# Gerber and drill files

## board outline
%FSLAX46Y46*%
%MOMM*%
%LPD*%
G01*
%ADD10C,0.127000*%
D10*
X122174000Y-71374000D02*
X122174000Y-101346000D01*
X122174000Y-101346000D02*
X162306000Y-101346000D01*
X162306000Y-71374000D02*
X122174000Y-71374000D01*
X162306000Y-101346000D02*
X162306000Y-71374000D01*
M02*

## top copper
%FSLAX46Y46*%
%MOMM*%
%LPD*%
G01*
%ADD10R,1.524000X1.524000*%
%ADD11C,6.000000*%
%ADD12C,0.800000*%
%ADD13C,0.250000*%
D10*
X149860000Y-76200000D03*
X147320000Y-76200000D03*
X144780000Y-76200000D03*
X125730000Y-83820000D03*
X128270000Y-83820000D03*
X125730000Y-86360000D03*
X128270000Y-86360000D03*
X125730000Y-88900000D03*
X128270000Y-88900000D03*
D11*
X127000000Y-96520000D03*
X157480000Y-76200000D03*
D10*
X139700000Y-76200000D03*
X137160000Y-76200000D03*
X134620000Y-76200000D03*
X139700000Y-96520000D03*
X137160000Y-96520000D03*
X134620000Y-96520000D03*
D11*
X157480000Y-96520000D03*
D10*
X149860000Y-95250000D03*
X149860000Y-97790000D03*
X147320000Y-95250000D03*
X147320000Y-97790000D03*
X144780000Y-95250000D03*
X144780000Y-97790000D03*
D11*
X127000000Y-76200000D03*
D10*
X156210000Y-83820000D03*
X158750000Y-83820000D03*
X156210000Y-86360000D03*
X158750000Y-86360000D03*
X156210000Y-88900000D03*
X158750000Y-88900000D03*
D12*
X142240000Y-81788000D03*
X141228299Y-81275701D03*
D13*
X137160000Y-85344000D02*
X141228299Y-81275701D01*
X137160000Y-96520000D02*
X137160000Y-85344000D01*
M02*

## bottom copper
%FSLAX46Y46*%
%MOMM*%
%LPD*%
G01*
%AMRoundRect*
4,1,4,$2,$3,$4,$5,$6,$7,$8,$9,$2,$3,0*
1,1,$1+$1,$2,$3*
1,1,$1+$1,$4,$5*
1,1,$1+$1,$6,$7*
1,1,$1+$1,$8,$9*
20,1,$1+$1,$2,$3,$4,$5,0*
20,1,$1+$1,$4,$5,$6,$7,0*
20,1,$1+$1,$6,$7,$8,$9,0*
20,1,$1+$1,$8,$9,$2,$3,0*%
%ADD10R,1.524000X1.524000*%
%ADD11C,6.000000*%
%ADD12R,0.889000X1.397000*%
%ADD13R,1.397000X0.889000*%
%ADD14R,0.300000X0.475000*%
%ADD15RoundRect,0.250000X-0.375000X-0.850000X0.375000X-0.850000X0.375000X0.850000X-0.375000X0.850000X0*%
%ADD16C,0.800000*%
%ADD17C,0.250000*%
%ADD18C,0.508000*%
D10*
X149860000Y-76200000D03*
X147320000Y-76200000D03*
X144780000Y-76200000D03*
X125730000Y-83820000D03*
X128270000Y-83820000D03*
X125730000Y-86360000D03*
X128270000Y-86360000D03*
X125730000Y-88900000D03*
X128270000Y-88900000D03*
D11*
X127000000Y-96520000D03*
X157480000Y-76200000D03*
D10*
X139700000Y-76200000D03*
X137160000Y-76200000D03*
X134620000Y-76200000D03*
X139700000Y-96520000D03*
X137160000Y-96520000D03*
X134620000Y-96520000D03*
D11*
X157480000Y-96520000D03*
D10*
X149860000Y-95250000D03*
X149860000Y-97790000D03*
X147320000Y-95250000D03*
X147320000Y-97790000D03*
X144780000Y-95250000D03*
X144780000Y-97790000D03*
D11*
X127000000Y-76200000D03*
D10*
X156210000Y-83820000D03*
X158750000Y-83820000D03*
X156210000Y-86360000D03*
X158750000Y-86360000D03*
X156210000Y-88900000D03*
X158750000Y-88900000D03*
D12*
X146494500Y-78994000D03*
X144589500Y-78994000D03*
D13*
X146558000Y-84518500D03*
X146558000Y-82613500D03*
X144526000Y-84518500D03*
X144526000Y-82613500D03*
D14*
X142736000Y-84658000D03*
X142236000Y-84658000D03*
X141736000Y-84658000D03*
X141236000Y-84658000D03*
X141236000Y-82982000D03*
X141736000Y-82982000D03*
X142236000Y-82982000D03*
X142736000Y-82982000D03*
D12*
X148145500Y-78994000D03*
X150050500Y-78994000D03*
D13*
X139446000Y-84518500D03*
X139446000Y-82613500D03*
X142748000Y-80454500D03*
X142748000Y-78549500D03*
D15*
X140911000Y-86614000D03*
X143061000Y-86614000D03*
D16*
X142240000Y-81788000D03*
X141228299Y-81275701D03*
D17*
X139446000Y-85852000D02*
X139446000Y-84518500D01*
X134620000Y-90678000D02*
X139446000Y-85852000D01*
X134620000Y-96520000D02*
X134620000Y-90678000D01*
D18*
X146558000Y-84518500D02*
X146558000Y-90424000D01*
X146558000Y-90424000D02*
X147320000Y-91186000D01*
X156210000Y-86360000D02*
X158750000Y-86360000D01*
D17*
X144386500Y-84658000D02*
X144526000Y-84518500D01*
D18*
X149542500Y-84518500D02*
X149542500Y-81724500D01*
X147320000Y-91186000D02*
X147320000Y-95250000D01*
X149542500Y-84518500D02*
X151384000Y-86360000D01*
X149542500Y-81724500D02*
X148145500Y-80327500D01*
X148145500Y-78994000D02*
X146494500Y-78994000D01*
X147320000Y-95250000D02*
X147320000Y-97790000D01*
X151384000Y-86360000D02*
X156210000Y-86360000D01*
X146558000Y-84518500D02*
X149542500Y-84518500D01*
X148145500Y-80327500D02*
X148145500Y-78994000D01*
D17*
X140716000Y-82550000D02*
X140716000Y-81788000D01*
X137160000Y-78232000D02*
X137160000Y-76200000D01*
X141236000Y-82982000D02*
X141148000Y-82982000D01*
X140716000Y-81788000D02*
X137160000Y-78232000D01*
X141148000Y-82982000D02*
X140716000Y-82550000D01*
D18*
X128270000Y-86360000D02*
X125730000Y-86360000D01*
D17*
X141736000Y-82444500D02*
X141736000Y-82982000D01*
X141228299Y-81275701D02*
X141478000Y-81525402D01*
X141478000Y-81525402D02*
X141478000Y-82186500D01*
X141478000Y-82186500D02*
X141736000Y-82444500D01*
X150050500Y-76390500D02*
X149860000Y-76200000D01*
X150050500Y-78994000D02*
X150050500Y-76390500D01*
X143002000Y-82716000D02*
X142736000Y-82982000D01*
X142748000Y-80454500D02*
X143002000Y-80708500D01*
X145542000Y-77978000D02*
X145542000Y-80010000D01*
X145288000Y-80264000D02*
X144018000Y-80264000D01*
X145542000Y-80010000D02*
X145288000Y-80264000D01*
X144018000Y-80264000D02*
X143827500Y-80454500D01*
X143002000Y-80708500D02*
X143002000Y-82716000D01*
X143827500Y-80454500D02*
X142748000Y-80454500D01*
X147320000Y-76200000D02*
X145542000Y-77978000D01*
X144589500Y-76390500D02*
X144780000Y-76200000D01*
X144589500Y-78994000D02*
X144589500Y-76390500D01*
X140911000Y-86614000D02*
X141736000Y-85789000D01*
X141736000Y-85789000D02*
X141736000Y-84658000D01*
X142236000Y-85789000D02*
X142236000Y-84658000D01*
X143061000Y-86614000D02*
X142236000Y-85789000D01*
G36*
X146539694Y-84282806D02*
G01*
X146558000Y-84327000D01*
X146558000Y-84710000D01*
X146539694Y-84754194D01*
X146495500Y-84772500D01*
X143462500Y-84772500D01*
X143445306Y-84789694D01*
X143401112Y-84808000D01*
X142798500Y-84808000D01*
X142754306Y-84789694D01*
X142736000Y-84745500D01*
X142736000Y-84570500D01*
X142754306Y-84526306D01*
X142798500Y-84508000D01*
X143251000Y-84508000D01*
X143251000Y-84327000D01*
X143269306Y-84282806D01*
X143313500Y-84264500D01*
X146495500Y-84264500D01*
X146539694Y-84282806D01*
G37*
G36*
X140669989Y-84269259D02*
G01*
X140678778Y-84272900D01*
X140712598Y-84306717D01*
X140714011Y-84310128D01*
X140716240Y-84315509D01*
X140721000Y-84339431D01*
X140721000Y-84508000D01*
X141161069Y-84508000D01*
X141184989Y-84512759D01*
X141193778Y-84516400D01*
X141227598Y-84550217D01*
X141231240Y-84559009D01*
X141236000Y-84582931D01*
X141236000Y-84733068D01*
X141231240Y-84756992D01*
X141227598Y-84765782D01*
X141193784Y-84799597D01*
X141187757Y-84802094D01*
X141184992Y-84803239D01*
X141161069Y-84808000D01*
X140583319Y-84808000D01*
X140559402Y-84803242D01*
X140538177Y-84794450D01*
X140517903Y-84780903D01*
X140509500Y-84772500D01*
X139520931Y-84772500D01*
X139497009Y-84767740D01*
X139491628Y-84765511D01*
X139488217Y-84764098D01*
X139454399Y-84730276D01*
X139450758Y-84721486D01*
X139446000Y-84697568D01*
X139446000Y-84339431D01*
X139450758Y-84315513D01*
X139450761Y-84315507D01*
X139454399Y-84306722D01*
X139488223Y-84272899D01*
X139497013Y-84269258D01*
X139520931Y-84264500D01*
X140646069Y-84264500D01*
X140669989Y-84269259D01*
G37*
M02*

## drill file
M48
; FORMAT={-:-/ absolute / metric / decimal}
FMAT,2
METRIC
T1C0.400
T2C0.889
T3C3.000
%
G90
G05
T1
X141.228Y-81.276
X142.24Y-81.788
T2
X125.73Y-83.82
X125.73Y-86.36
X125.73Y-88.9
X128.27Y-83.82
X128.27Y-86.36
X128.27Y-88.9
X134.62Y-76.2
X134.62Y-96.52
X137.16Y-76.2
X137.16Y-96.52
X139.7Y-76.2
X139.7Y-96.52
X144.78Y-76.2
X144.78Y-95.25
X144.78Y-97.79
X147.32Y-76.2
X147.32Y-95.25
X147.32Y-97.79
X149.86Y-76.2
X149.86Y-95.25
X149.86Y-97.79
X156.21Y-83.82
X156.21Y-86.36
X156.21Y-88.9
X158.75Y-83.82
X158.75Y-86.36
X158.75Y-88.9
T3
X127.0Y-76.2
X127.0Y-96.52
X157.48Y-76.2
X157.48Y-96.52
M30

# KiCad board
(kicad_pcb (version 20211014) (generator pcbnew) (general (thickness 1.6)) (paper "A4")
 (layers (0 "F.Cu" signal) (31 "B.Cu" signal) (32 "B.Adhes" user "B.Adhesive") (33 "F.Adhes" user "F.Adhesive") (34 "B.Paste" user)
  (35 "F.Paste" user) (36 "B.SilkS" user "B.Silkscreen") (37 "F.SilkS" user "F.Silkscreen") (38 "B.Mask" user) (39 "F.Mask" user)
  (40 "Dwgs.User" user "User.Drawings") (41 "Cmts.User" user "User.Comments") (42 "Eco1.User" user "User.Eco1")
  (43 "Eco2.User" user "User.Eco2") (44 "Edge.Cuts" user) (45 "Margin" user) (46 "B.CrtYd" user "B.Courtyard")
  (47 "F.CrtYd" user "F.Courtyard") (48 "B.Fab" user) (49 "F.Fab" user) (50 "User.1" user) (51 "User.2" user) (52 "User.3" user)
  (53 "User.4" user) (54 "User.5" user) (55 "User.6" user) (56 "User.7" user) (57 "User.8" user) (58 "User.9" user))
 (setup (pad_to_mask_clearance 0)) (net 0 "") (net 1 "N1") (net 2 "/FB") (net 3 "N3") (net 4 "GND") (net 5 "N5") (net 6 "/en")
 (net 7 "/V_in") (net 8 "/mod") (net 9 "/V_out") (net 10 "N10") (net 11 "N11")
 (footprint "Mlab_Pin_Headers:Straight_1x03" (layer "F.Cu") (at 147.32 76.2 -90)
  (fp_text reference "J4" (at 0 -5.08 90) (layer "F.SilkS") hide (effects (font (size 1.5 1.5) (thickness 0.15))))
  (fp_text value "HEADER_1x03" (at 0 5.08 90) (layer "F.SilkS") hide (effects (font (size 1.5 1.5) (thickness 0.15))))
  (pad "1" thru_hole rect (at 0 -2.54 270) (size 1.524 1.524) (drill 0.889) (layers *.Cu *.Mask) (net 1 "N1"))
  (pad "2" thru_hole rect (at 0 0 270) (size 1.524 1.524) (drill 0.889) (layers *.Cu *.Mask) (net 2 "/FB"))
  (pad "3" thru_hole rect (at 0 2.54 270) (size 1.524 1.524) (drill 0.889) (layers *.Cu *.Mask) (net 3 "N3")))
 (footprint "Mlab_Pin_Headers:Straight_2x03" (layer "F.Cu") (at 127 86.36)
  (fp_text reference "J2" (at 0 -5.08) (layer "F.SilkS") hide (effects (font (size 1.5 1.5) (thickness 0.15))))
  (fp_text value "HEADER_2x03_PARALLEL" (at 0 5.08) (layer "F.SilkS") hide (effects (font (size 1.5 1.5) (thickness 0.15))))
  (pad "1" thru_hole rect (at -1.27 -2.54) (size 1.524 1.524) (drill 0.889) (layers *.Cu *.Mask) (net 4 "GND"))
  (pad "2" thru_hole rect (at 1.27 -2.54) (size 1.524 1.524) (drill 0.889) (layers *.Cu *.Mask) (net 4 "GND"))
  (pad "3" thru_hole rect (at -1.27 0) (size 1.524 1.524) (drill 0.889) (layers *.Cu *.Mask) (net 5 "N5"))
  (pad "4" thru_hole rect (at 1.27 0) (size 1.524 1.524) (drill 0.889) (layers *.Cu *.Mask) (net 5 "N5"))
  (pad "5" thru_hole rect (at -1.27 2.54) (size 1.524 1.524) (drill 0.889) (layers *.Cu *.Mask) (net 4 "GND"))
  (pad "6" thru_hole rect (at 1.27 2.54) (size 1.524 1.524) (drill 0.889) (layers *.Cu *.Mask) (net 4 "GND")))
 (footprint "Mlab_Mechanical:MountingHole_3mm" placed (layer "F.Cu") (at 127 96.52)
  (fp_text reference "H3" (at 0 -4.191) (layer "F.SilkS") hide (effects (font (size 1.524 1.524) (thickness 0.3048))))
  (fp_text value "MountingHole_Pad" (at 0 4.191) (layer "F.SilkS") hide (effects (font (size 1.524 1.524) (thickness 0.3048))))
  (pad "1" thru_hole circle (at 0 0) (size 6 6) (drill 3) (layers *.Cu *.Mask) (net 4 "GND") (clearance 1) (zone_connect 2)))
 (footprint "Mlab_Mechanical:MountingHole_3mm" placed (layer "F.Cu") (at 157.48 76.2)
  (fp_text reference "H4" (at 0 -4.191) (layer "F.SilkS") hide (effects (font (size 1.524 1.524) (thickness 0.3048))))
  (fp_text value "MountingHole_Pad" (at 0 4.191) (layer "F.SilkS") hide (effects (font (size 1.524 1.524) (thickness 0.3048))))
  (pad "1" thru_hole circle (at 0 0) (size 6 6) (drill 3) (layers *.Cu *.Mask) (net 4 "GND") (clearance 1) (zone_connect 2)))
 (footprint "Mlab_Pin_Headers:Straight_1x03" (layer "F.Cu") (at 137.16 76.2 -90)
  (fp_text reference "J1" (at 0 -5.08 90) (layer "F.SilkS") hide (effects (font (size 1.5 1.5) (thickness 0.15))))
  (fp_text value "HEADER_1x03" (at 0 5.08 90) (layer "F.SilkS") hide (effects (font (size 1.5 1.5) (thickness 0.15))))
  (pad "1" thru_hole rect (at 0 -2.54 270) (size 1.524 1.524) (drill 0.889) (layers *.Cu *.Mask) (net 4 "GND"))
  (pad "2" thru_hole rect (at 0 0 270) (size 1.524 1.524) (drill 0.889) (layers *.Cu *.Mask) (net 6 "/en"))
  (pad "3" thru_hole rect (at 0 2.54 270) (size 1.524 1.524) (drill 0.889) (layers *.Cu *.Mask) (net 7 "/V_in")))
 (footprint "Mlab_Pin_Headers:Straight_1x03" (layer "F.Cu") (at 137.16 96.52 -90)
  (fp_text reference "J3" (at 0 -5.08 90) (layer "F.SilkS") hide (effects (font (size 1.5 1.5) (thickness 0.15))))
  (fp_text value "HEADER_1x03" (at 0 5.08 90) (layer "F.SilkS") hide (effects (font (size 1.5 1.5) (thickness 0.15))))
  (pad "1" thru_hole rect (at 0 -2.54 270) (size 1.524 1.524) (drill 0.889) (layers *.Cu *.Mask) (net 4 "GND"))
  (pad "2" thru_hole rect (at 0 0 270) (size 1.524 1.524) (drill 0.889) (layers *.Cu *.Mask) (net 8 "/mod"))
  (pad "3" thru_hole rect (at 0 2.54 270) (size 1.524 1.524) (drill 0.889) (layers *.Cu *.Mask) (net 7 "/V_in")))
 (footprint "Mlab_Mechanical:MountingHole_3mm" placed (layer "F.Cu") (at 157.48 96.52)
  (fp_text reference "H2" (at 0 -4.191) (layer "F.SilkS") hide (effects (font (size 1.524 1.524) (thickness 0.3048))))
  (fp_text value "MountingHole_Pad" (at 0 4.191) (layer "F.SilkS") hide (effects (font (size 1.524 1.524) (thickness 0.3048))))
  (pad "1" thru_hole circle (at 0 0) (size 6 6) (drill 3) (layers *.Cu *.Mask) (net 4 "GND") (clearance 1) (zone_connect 2)))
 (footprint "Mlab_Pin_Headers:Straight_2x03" (layer "F.Cu") (at 147.32 96.52 -90)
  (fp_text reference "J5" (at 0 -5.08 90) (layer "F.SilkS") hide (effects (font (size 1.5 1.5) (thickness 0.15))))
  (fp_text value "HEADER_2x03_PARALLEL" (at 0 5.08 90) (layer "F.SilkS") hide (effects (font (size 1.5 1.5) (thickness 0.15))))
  (pad "1" thru_hole rect (at -1.27 -2.54 270) (size 1.524 1.524) (drill 0.889) (layers *.Cu *.Mask) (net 4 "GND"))
  (pad "2" thru_hole rect (at 1.27 -2.54 270) (size 1.524 1.524) (drill 0.889) (layers *.Cu *.Mask) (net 4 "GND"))
  (pad "3" thru_hole rect (at -1.27 0 270) (size 1.524 1.524) (drill 0.889) (layers *.Cu *.Mask) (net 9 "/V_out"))
  (pad "4" thru_hole rect (at 1.27 0 270) (size 1.524 1.524) (drill 0.889) (layers *.Cu *.Mask) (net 9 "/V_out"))
  (pad "5" thru_hole rect (at -1.27 2.54 270) (size 1.524 1.524) (drill 0.889) (layers *.Cu *.Mask) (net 4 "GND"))
  (pad "6" thru_hole rect (at 1.27 2.54 270) (size 1.524 1.524) (drill 0.889) (layers *.Cu *.Mask) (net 4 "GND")))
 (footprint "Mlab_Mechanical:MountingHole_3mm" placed (layer "F.Cu") (at 127 76.2)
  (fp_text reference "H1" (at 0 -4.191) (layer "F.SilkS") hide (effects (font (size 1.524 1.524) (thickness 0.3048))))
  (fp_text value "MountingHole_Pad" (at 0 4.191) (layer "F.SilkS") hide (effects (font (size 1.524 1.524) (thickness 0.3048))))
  (pad "1" thru_hole circle (at 0 0) (size 6 6) (drill 3) (layers *.Cu *.Mask) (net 4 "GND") (clearance 1) (zone_connect 2)))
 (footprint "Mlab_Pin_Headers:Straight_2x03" (layer "F.Cu") (at 157.48 86.36)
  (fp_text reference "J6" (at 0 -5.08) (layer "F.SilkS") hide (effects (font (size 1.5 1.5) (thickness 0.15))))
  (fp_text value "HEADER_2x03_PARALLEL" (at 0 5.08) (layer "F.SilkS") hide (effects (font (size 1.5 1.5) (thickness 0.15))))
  (pad "1" thru_hole rect (at -1.27 -2.54) (size 1.524 1.524) (drill 0.889) (layers *.Cu *.Mask) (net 4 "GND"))
  (pad "2" thru_hole rect (at 1.27 -2.54) (size 1.524 1.524) (drill 0.889) (layers *.Cu *.Mask) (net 4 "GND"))
  (pad "3" thru_hole rect (at -1.27 0) (size 1.524 1.524) (drill 0.889) (layers *.Cu *.Mask) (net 9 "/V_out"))
  (pad "4" thru_hole rect (at 1.27 0) (size 1.524 1.524) (drill 0.889) (layers *.Cu *.Mask) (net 9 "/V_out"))
  (pad "5" thru_hole rect (at -1.27 2.54) (size 1.524 1.524) (drill 0.889) (layers *.Cu *.Mask) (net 4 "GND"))
  (pad "6" thru_hole rect (at 1.27 2.54) (size 1.524 1.524) (drill 0.889) (layers *.Cu *.Mask) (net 4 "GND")))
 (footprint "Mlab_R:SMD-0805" (layer "B.Cu") (at 145.542 78.994 180)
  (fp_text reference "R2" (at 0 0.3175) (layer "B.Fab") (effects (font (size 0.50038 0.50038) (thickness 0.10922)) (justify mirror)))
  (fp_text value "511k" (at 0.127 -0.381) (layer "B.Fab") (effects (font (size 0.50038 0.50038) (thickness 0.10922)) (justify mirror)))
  (pad "1" smd rect locked (at -0.9525 0 180) (size 0.889 1.397) (layers "B.Cu" "B.Paste" "B.Mask") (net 9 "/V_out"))
  (pad "2" smd rect locked (at 0.9525 0 180) (size 0.889 1.397) (layers "B.Cu" "B.Paste" "B.Mask") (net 3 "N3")))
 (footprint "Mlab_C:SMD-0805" (layer "B.Cu") (at 146.558 83.566 90)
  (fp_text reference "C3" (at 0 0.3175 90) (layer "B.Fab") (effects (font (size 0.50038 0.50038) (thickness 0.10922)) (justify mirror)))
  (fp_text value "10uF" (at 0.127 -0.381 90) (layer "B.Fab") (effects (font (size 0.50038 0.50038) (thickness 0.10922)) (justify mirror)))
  (pad "1" smd rect locked (at -0.9525 0 90) (size 0.889 1.397) (layers "B.Cu" "B.Paste" "B.Mask") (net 9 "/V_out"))
  (pad "2" smd rect locked (at 0.9525 0 90) (size 0.889 1.397) (layers "B.Cu" "B.Paste" "B.Mask") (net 4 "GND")))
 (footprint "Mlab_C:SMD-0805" (layer "B.Cu") (at 144.526 83.566 90)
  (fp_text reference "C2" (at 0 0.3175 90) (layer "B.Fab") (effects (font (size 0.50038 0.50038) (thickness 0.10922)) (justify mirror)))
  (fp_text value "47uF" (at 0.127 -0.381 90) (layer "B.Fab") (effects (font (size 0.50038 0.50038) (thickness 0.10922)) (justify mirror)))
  (pad "1" smd rect locked (at -0.9525 0 90) (size 0.889 1.397) (layers "B.Cu" "B.Paste" "B.Mask") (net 9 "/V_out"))
  (pad "2" smd rect locked (at 0.9525 0 90) (size 0.889 1.397) (layers "B.Cu" "B.Paste" "B.Mask") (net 4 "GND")))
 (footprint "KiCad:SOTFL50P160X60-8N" (layer "B.Cu") (at 141.986 83.82 90)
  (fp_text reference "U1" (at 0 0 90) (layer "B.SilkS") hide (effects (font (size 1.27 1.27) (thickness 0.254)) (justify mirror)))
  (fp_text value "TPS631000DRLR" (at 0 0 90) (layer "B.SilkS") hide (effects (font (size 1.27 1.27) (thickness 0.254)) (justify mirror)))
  (pad "1" smd rect locked (at -0.838 0.75) (size 0.3 0.475) (layers "B.Cu" "B.Paste" "B.Mask") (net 9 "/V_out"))
  (pad "2" smd rect locked (at -0.838 0.25) (size 0.3 0.475) (layers "B.Cu" "B.Paste" "B.Mask") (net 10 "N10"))
  (pad "3" smd rect locked (at -0.838 -0.25) (size 0.3 0.475) (layers "B.Cu" "B.Paste" "B.Mask") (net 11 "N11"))
  (pad "4" smd rect locked (at -0.838 -0.75) (size 0.3 0.475) (layers "B.Cu" "B.Paste" "B.Mask") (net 7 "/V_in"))
  (pad "5" smd rect locked (at 0.838 -0.75) (size 0.3 0.475) (layers "B.Cu" "B.Paste" "B.Mask") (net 6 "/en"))
  (pad "6" smd rect locked (at 0.838 -0.25) (size 0.3 0.475) (layers "B.Cu" "B.Paste" "B.Mask") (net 8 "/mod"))
  (pad "7" smd rect locked (at 0.838 0.25) (size 0.3 0.475) (layers "B.Cu" "B.Paste" "B.Mask") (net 4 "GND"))
  (pad "8" smd rect locked (at 0.838 0.75) (size 0.3 0.475) (layers "B.Cu" "B.Paste" "B.Mask") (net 2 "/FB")))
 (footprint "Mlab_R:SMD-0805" (layer "B.Cu") (at 149.098 78.994)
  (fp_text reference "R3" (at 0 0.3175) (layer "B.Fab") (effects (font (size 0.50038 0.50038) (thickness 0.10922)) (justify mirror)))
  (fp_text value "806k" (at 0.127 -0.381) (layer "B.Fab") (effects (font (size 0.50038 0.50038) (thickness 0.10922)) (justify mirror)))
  (pad "1" smd rect locked (at -0.9525 0) (size 0.889 1.397) (layers "B.Cu" "B.Paste" "B.Mask") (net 9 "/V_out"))
  (pad "2" smd rect locked (at 0.9525 0) (size 0.889 1.397) (layers "B.Cu" "B.Paste" "B.Mask") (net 1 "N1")))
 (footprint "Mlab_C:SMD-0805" (layer "B.Cu") (at 139.446 83.566 90)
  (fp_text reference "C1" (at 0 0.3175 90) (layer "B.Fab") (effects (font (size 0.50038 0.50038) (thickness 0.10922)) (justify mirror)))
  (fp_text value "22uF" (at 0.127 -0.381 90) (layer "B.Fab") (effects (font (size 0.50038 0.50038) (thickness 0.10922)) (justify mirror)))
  (pad "1" smd rect locked (at -0.9525 0 90) (size 0.889 1.397) (layers "B.Cu" "B.Paste" "B.Mask") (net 7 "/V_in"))
  (pad "2" smd rect locked (at 0.9525 0 90) (size 0.889 1.397) (layers "B.Cu" "B.Paste" "B.Mask") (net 4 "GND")))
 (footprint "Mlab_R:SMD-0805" (layer "B.Cu") (at 142.748 79.502 90)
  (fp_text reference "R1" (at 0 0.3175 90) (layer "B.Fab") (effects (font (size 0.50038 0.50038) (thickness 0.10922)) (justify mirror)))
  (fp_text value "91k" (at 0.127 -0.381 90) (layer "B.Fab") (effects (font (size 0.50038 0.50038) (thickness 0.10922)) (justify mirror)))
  (pad "1" smd rect locked (at -0.9525 0 90) (size 0.889 1.397) (layers "B.Cu" "B.Paste" "B.Mask") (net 2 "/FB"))
  (pad "2" smd rect locked (at 0.9525 0 90) (size 0.889 1.397) (layers "B.Cu" "B.Paste" "B.Mask") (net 4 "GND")))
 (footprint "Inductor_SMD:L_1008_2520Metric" (layer "B.Cu") (at 141.986 86.614)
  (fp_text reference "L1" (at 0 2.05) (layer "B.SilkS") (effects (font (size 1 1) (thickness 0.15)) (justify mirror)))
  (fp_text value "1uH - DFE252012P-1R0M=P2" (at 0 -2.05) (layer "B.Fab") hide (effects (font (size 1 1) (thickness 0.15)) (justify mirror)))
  (pad "1" smd roundrect (at -1.075 0) (size 1.25 2.2) (layers "B.Cu" "B.Paste" "B.Mask") (roundrect_rratio 0.2) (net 11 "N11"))
  (pad "2" smd roundrect (at 1.075 0) (size 1.25 2.2) (layers "B.Cu" "B.Paste" "B.Mask") (roundrect_rratio 0.2) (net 10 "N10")))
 (gr_line (start 122.174 71.374) (end 122.174 101.346) (layer "Edge.Cuts") (width 0.127))
 (gr_line (start 122.174 101.346) (end 162.306 101.346) (layer "Edge.Cuts") (width 0.127))
 (gr_line (start 162.306 71.374) (end 122.174 71.374) (layer "Edge.Cuts") (width 0.127))
 (gr_line (start 162.306 101.346) (end 162.306 71.374) (layer "Edge.Cuts") (width 0.127))
 (via (at 142.24 81.788) (size 0.8) (drill 0.4) (layers "F.Cu" "B.Cu") (free) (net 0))
 (segment (start 139.446 85.852) (end 139.446 84.5185) (width 0.25) (layer "B.Cu") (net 7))
 (segment (start 134.62 90.678) (end 139.446 85.852) (width 0.25) (layer "B.Cu") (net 7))
 (segment (start 134.62 96.52) (end 134.62 90.678) (width 0.25) (layer "B.Cu") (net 7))
 (segment (start 146.558 84.5185) (end 146.558 90.424) (width 0.508) (layer "B.Cu") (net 9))
 (segment (start 146.558 90.424) (end 147.32 91.186) (width 0.508) (layer "B.Cu") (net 9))
 (segment (start 156.21 86.36) (end 158.75 86.36) (width 0.508) (layer "B.Cu") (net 9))
 (segment (start 144.3865 84.658) (end 144.526 84.5185) (width 0.25) (layer "B.Cu") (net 9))
 (segment (start 149.5425 84.5185) (end 149.5425 81.7245) (width 0.508) (layer "B.Cu") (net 9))
 (segment (start 147.32 91.186) (end 147.32 95.25) (width 0.508) (layer "B.Cu") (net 9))
 (segment (start 149.5425 84.5185) (end 151.384 86.36) (width 0.508) (layer "B.Cu") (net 9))
 (segment (start 149.5425 81.7245) (end 148.1455 80.3275) (width 0.508) (layer "B.Cu") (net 9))
 (segment (start 148.1455 78.994) (end 146.4945 78.994) (width 0.508) (layer "B.Cu") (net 9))
 (segment (start 147.32 95.25) (end 147.32 97.79) (width 0.508) (layer "B.Cu") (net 9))
 (segment (start 151.384 86.36) (end 156.21 86.36) (width 0.508) (layer "B.Cu") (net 9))
 (segment (start 146.558 84.5185) (end 149.5425 84.5185) (width 0.508) (layer "B.Cu") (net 9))
 (segment (start 148.1455 80.3275) (end 148.1455 78.994) (width 0.508) (layer "B.Cu") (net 9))
 (segment (start 140.716 82.55) (end 140.716 81.788) (width 0.25) (layer "B.Cu") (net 6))
 (segment (start 137.16 78.232) (end 137.16 76.2) (width 0.25) (layer "B.Cu") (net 6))
 (segment (start 141.236 82.982) (end 141.148 82.982) (width 0.25) (layer "B.Cu") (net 6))
 (segment (start 140.716 81.788) (end 137.16 78.232) (width 0.25) (layer "B.Cu") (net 6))
 (segment (start 141.148 82.982) (end 140.716 82.55) (width 0.25) (layer "B.Cu") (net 6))
 (segment (start 128.27 86.36) (end 125.73 86.36) (width 0.508) (layer "B.Cu") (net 5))
 (segment (start 137.16 85.344) (end 141.228299 81.275701) (width 0.25) (layer "F.Cu") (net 8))
 (segment (start 137.16 96.52) (end 137.16 85.344) (width 0.25) (layer "F.Cu") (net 8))
 (via (at 141.228299 81.275701) (size 0.8) (drill 0.4) (layers "F.Cu" "B.Cu") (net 8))
 (segment (start 141.736 82.4445) (end 141.736 82.982) (width 0.25) (layer "B.Cu") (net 8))
 (segment (start 141.228299 81.275701) (end 141.478 81.525402) (width 0.25) (layer "B.Cu") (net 8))
 (segment (start 141.478 81.525402) (end 141.478 82.1865) (width 0.25) (layer "B.Cu") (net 8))
 (segment (start 141.478 82.1865) (end 141.736 82.4445) (width 0.25) (layer "B.Cu") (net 8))
 (segment (start 150.0505 76.3905) (end 149.86 76.2) (width 0.25) (layer "B.Cu") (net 1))
 (segment (start 150.0505 78.994) (end 150.0505 76.3905) (width 0.25) (layer "B.Cu") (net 1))
 (segment (start 143.002 82.716) (end 142.736 82.982) (width 0.25) (layer "B.Cu") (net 2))
 (segment (start 142.748 80.4545) (end 143.002 80.7085) (width 0.25) (layer "B.Cu") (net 2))
 (segment (start 145.542 77.978) (end 145.542 80.01) (width 0.25) (layer "B.Cu") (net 2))
 (segment (start 145.288 80.264) (end 144.018 80.264) (width 0.25) (layer "B.Cu") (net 2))
 (segment (start 145.542 80.01) (end 145.288 80.264) (width 0.25) (layer "B.Cu") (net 2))
 (segment (start 144.018 80.264) (end 143.8275 80.4545) (width 0.25) (layer "B.Cu") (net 2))
 (segment (start 143.002 80.7085) (end 143.002 82.716) (width 0.25) (layer "B.Cu") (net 2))
 (segment (start 143.8275 80.4545) (end 142.748 80.4545) (width 0.25) (layer "B.Cu") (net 2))
 (segment (start 147.32 76.2) (end 145.542 77.978) (width 0.25) (layer "B.Cu") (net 2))
 (segment (start 144.5895 76.3905) (end 144.78 76.2) (width 0.25) (layer "B.Cu") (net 3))
 (segment (start 144.5895 78.994) (end 144.5895 76.3905) (width 0.25) (layer "B.Cu") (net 3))
 (segment (start 140.911 86.614) (end 141.736 85.789) (width 0.25) (layer "B.Cu") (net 11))
 (segment (start 141.736 85.789) (end 141.736 84.658) (width 0.25) (layer "B.Cu") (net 11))
 (segment (start 142.236 85.789) (end 142.236 84.658) (width 0.25) (layer "B.Cu") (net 10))
 (segment (start 143.061 86.614) (end 142.236 85.789) (width 0.25) (layer "B.Cu") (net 10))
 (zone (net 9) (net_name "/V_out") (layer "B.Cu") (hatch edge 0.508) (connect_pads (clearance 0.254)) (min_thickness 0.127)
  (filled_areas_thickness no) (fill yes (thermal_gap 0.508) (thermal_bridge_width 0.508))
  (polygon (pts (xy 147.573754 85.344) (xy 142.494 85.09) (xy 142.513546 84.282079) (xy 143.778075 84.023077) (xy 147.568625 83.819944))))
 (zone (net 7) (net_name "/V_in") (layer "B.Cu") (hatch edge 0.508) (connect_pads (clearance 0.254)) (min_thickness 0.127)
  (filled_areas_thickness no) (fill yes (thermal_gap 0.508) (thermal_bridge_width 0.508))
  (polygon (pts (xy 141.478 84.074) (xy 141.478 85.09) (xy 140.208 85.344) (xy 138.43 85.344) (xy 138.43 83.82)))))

